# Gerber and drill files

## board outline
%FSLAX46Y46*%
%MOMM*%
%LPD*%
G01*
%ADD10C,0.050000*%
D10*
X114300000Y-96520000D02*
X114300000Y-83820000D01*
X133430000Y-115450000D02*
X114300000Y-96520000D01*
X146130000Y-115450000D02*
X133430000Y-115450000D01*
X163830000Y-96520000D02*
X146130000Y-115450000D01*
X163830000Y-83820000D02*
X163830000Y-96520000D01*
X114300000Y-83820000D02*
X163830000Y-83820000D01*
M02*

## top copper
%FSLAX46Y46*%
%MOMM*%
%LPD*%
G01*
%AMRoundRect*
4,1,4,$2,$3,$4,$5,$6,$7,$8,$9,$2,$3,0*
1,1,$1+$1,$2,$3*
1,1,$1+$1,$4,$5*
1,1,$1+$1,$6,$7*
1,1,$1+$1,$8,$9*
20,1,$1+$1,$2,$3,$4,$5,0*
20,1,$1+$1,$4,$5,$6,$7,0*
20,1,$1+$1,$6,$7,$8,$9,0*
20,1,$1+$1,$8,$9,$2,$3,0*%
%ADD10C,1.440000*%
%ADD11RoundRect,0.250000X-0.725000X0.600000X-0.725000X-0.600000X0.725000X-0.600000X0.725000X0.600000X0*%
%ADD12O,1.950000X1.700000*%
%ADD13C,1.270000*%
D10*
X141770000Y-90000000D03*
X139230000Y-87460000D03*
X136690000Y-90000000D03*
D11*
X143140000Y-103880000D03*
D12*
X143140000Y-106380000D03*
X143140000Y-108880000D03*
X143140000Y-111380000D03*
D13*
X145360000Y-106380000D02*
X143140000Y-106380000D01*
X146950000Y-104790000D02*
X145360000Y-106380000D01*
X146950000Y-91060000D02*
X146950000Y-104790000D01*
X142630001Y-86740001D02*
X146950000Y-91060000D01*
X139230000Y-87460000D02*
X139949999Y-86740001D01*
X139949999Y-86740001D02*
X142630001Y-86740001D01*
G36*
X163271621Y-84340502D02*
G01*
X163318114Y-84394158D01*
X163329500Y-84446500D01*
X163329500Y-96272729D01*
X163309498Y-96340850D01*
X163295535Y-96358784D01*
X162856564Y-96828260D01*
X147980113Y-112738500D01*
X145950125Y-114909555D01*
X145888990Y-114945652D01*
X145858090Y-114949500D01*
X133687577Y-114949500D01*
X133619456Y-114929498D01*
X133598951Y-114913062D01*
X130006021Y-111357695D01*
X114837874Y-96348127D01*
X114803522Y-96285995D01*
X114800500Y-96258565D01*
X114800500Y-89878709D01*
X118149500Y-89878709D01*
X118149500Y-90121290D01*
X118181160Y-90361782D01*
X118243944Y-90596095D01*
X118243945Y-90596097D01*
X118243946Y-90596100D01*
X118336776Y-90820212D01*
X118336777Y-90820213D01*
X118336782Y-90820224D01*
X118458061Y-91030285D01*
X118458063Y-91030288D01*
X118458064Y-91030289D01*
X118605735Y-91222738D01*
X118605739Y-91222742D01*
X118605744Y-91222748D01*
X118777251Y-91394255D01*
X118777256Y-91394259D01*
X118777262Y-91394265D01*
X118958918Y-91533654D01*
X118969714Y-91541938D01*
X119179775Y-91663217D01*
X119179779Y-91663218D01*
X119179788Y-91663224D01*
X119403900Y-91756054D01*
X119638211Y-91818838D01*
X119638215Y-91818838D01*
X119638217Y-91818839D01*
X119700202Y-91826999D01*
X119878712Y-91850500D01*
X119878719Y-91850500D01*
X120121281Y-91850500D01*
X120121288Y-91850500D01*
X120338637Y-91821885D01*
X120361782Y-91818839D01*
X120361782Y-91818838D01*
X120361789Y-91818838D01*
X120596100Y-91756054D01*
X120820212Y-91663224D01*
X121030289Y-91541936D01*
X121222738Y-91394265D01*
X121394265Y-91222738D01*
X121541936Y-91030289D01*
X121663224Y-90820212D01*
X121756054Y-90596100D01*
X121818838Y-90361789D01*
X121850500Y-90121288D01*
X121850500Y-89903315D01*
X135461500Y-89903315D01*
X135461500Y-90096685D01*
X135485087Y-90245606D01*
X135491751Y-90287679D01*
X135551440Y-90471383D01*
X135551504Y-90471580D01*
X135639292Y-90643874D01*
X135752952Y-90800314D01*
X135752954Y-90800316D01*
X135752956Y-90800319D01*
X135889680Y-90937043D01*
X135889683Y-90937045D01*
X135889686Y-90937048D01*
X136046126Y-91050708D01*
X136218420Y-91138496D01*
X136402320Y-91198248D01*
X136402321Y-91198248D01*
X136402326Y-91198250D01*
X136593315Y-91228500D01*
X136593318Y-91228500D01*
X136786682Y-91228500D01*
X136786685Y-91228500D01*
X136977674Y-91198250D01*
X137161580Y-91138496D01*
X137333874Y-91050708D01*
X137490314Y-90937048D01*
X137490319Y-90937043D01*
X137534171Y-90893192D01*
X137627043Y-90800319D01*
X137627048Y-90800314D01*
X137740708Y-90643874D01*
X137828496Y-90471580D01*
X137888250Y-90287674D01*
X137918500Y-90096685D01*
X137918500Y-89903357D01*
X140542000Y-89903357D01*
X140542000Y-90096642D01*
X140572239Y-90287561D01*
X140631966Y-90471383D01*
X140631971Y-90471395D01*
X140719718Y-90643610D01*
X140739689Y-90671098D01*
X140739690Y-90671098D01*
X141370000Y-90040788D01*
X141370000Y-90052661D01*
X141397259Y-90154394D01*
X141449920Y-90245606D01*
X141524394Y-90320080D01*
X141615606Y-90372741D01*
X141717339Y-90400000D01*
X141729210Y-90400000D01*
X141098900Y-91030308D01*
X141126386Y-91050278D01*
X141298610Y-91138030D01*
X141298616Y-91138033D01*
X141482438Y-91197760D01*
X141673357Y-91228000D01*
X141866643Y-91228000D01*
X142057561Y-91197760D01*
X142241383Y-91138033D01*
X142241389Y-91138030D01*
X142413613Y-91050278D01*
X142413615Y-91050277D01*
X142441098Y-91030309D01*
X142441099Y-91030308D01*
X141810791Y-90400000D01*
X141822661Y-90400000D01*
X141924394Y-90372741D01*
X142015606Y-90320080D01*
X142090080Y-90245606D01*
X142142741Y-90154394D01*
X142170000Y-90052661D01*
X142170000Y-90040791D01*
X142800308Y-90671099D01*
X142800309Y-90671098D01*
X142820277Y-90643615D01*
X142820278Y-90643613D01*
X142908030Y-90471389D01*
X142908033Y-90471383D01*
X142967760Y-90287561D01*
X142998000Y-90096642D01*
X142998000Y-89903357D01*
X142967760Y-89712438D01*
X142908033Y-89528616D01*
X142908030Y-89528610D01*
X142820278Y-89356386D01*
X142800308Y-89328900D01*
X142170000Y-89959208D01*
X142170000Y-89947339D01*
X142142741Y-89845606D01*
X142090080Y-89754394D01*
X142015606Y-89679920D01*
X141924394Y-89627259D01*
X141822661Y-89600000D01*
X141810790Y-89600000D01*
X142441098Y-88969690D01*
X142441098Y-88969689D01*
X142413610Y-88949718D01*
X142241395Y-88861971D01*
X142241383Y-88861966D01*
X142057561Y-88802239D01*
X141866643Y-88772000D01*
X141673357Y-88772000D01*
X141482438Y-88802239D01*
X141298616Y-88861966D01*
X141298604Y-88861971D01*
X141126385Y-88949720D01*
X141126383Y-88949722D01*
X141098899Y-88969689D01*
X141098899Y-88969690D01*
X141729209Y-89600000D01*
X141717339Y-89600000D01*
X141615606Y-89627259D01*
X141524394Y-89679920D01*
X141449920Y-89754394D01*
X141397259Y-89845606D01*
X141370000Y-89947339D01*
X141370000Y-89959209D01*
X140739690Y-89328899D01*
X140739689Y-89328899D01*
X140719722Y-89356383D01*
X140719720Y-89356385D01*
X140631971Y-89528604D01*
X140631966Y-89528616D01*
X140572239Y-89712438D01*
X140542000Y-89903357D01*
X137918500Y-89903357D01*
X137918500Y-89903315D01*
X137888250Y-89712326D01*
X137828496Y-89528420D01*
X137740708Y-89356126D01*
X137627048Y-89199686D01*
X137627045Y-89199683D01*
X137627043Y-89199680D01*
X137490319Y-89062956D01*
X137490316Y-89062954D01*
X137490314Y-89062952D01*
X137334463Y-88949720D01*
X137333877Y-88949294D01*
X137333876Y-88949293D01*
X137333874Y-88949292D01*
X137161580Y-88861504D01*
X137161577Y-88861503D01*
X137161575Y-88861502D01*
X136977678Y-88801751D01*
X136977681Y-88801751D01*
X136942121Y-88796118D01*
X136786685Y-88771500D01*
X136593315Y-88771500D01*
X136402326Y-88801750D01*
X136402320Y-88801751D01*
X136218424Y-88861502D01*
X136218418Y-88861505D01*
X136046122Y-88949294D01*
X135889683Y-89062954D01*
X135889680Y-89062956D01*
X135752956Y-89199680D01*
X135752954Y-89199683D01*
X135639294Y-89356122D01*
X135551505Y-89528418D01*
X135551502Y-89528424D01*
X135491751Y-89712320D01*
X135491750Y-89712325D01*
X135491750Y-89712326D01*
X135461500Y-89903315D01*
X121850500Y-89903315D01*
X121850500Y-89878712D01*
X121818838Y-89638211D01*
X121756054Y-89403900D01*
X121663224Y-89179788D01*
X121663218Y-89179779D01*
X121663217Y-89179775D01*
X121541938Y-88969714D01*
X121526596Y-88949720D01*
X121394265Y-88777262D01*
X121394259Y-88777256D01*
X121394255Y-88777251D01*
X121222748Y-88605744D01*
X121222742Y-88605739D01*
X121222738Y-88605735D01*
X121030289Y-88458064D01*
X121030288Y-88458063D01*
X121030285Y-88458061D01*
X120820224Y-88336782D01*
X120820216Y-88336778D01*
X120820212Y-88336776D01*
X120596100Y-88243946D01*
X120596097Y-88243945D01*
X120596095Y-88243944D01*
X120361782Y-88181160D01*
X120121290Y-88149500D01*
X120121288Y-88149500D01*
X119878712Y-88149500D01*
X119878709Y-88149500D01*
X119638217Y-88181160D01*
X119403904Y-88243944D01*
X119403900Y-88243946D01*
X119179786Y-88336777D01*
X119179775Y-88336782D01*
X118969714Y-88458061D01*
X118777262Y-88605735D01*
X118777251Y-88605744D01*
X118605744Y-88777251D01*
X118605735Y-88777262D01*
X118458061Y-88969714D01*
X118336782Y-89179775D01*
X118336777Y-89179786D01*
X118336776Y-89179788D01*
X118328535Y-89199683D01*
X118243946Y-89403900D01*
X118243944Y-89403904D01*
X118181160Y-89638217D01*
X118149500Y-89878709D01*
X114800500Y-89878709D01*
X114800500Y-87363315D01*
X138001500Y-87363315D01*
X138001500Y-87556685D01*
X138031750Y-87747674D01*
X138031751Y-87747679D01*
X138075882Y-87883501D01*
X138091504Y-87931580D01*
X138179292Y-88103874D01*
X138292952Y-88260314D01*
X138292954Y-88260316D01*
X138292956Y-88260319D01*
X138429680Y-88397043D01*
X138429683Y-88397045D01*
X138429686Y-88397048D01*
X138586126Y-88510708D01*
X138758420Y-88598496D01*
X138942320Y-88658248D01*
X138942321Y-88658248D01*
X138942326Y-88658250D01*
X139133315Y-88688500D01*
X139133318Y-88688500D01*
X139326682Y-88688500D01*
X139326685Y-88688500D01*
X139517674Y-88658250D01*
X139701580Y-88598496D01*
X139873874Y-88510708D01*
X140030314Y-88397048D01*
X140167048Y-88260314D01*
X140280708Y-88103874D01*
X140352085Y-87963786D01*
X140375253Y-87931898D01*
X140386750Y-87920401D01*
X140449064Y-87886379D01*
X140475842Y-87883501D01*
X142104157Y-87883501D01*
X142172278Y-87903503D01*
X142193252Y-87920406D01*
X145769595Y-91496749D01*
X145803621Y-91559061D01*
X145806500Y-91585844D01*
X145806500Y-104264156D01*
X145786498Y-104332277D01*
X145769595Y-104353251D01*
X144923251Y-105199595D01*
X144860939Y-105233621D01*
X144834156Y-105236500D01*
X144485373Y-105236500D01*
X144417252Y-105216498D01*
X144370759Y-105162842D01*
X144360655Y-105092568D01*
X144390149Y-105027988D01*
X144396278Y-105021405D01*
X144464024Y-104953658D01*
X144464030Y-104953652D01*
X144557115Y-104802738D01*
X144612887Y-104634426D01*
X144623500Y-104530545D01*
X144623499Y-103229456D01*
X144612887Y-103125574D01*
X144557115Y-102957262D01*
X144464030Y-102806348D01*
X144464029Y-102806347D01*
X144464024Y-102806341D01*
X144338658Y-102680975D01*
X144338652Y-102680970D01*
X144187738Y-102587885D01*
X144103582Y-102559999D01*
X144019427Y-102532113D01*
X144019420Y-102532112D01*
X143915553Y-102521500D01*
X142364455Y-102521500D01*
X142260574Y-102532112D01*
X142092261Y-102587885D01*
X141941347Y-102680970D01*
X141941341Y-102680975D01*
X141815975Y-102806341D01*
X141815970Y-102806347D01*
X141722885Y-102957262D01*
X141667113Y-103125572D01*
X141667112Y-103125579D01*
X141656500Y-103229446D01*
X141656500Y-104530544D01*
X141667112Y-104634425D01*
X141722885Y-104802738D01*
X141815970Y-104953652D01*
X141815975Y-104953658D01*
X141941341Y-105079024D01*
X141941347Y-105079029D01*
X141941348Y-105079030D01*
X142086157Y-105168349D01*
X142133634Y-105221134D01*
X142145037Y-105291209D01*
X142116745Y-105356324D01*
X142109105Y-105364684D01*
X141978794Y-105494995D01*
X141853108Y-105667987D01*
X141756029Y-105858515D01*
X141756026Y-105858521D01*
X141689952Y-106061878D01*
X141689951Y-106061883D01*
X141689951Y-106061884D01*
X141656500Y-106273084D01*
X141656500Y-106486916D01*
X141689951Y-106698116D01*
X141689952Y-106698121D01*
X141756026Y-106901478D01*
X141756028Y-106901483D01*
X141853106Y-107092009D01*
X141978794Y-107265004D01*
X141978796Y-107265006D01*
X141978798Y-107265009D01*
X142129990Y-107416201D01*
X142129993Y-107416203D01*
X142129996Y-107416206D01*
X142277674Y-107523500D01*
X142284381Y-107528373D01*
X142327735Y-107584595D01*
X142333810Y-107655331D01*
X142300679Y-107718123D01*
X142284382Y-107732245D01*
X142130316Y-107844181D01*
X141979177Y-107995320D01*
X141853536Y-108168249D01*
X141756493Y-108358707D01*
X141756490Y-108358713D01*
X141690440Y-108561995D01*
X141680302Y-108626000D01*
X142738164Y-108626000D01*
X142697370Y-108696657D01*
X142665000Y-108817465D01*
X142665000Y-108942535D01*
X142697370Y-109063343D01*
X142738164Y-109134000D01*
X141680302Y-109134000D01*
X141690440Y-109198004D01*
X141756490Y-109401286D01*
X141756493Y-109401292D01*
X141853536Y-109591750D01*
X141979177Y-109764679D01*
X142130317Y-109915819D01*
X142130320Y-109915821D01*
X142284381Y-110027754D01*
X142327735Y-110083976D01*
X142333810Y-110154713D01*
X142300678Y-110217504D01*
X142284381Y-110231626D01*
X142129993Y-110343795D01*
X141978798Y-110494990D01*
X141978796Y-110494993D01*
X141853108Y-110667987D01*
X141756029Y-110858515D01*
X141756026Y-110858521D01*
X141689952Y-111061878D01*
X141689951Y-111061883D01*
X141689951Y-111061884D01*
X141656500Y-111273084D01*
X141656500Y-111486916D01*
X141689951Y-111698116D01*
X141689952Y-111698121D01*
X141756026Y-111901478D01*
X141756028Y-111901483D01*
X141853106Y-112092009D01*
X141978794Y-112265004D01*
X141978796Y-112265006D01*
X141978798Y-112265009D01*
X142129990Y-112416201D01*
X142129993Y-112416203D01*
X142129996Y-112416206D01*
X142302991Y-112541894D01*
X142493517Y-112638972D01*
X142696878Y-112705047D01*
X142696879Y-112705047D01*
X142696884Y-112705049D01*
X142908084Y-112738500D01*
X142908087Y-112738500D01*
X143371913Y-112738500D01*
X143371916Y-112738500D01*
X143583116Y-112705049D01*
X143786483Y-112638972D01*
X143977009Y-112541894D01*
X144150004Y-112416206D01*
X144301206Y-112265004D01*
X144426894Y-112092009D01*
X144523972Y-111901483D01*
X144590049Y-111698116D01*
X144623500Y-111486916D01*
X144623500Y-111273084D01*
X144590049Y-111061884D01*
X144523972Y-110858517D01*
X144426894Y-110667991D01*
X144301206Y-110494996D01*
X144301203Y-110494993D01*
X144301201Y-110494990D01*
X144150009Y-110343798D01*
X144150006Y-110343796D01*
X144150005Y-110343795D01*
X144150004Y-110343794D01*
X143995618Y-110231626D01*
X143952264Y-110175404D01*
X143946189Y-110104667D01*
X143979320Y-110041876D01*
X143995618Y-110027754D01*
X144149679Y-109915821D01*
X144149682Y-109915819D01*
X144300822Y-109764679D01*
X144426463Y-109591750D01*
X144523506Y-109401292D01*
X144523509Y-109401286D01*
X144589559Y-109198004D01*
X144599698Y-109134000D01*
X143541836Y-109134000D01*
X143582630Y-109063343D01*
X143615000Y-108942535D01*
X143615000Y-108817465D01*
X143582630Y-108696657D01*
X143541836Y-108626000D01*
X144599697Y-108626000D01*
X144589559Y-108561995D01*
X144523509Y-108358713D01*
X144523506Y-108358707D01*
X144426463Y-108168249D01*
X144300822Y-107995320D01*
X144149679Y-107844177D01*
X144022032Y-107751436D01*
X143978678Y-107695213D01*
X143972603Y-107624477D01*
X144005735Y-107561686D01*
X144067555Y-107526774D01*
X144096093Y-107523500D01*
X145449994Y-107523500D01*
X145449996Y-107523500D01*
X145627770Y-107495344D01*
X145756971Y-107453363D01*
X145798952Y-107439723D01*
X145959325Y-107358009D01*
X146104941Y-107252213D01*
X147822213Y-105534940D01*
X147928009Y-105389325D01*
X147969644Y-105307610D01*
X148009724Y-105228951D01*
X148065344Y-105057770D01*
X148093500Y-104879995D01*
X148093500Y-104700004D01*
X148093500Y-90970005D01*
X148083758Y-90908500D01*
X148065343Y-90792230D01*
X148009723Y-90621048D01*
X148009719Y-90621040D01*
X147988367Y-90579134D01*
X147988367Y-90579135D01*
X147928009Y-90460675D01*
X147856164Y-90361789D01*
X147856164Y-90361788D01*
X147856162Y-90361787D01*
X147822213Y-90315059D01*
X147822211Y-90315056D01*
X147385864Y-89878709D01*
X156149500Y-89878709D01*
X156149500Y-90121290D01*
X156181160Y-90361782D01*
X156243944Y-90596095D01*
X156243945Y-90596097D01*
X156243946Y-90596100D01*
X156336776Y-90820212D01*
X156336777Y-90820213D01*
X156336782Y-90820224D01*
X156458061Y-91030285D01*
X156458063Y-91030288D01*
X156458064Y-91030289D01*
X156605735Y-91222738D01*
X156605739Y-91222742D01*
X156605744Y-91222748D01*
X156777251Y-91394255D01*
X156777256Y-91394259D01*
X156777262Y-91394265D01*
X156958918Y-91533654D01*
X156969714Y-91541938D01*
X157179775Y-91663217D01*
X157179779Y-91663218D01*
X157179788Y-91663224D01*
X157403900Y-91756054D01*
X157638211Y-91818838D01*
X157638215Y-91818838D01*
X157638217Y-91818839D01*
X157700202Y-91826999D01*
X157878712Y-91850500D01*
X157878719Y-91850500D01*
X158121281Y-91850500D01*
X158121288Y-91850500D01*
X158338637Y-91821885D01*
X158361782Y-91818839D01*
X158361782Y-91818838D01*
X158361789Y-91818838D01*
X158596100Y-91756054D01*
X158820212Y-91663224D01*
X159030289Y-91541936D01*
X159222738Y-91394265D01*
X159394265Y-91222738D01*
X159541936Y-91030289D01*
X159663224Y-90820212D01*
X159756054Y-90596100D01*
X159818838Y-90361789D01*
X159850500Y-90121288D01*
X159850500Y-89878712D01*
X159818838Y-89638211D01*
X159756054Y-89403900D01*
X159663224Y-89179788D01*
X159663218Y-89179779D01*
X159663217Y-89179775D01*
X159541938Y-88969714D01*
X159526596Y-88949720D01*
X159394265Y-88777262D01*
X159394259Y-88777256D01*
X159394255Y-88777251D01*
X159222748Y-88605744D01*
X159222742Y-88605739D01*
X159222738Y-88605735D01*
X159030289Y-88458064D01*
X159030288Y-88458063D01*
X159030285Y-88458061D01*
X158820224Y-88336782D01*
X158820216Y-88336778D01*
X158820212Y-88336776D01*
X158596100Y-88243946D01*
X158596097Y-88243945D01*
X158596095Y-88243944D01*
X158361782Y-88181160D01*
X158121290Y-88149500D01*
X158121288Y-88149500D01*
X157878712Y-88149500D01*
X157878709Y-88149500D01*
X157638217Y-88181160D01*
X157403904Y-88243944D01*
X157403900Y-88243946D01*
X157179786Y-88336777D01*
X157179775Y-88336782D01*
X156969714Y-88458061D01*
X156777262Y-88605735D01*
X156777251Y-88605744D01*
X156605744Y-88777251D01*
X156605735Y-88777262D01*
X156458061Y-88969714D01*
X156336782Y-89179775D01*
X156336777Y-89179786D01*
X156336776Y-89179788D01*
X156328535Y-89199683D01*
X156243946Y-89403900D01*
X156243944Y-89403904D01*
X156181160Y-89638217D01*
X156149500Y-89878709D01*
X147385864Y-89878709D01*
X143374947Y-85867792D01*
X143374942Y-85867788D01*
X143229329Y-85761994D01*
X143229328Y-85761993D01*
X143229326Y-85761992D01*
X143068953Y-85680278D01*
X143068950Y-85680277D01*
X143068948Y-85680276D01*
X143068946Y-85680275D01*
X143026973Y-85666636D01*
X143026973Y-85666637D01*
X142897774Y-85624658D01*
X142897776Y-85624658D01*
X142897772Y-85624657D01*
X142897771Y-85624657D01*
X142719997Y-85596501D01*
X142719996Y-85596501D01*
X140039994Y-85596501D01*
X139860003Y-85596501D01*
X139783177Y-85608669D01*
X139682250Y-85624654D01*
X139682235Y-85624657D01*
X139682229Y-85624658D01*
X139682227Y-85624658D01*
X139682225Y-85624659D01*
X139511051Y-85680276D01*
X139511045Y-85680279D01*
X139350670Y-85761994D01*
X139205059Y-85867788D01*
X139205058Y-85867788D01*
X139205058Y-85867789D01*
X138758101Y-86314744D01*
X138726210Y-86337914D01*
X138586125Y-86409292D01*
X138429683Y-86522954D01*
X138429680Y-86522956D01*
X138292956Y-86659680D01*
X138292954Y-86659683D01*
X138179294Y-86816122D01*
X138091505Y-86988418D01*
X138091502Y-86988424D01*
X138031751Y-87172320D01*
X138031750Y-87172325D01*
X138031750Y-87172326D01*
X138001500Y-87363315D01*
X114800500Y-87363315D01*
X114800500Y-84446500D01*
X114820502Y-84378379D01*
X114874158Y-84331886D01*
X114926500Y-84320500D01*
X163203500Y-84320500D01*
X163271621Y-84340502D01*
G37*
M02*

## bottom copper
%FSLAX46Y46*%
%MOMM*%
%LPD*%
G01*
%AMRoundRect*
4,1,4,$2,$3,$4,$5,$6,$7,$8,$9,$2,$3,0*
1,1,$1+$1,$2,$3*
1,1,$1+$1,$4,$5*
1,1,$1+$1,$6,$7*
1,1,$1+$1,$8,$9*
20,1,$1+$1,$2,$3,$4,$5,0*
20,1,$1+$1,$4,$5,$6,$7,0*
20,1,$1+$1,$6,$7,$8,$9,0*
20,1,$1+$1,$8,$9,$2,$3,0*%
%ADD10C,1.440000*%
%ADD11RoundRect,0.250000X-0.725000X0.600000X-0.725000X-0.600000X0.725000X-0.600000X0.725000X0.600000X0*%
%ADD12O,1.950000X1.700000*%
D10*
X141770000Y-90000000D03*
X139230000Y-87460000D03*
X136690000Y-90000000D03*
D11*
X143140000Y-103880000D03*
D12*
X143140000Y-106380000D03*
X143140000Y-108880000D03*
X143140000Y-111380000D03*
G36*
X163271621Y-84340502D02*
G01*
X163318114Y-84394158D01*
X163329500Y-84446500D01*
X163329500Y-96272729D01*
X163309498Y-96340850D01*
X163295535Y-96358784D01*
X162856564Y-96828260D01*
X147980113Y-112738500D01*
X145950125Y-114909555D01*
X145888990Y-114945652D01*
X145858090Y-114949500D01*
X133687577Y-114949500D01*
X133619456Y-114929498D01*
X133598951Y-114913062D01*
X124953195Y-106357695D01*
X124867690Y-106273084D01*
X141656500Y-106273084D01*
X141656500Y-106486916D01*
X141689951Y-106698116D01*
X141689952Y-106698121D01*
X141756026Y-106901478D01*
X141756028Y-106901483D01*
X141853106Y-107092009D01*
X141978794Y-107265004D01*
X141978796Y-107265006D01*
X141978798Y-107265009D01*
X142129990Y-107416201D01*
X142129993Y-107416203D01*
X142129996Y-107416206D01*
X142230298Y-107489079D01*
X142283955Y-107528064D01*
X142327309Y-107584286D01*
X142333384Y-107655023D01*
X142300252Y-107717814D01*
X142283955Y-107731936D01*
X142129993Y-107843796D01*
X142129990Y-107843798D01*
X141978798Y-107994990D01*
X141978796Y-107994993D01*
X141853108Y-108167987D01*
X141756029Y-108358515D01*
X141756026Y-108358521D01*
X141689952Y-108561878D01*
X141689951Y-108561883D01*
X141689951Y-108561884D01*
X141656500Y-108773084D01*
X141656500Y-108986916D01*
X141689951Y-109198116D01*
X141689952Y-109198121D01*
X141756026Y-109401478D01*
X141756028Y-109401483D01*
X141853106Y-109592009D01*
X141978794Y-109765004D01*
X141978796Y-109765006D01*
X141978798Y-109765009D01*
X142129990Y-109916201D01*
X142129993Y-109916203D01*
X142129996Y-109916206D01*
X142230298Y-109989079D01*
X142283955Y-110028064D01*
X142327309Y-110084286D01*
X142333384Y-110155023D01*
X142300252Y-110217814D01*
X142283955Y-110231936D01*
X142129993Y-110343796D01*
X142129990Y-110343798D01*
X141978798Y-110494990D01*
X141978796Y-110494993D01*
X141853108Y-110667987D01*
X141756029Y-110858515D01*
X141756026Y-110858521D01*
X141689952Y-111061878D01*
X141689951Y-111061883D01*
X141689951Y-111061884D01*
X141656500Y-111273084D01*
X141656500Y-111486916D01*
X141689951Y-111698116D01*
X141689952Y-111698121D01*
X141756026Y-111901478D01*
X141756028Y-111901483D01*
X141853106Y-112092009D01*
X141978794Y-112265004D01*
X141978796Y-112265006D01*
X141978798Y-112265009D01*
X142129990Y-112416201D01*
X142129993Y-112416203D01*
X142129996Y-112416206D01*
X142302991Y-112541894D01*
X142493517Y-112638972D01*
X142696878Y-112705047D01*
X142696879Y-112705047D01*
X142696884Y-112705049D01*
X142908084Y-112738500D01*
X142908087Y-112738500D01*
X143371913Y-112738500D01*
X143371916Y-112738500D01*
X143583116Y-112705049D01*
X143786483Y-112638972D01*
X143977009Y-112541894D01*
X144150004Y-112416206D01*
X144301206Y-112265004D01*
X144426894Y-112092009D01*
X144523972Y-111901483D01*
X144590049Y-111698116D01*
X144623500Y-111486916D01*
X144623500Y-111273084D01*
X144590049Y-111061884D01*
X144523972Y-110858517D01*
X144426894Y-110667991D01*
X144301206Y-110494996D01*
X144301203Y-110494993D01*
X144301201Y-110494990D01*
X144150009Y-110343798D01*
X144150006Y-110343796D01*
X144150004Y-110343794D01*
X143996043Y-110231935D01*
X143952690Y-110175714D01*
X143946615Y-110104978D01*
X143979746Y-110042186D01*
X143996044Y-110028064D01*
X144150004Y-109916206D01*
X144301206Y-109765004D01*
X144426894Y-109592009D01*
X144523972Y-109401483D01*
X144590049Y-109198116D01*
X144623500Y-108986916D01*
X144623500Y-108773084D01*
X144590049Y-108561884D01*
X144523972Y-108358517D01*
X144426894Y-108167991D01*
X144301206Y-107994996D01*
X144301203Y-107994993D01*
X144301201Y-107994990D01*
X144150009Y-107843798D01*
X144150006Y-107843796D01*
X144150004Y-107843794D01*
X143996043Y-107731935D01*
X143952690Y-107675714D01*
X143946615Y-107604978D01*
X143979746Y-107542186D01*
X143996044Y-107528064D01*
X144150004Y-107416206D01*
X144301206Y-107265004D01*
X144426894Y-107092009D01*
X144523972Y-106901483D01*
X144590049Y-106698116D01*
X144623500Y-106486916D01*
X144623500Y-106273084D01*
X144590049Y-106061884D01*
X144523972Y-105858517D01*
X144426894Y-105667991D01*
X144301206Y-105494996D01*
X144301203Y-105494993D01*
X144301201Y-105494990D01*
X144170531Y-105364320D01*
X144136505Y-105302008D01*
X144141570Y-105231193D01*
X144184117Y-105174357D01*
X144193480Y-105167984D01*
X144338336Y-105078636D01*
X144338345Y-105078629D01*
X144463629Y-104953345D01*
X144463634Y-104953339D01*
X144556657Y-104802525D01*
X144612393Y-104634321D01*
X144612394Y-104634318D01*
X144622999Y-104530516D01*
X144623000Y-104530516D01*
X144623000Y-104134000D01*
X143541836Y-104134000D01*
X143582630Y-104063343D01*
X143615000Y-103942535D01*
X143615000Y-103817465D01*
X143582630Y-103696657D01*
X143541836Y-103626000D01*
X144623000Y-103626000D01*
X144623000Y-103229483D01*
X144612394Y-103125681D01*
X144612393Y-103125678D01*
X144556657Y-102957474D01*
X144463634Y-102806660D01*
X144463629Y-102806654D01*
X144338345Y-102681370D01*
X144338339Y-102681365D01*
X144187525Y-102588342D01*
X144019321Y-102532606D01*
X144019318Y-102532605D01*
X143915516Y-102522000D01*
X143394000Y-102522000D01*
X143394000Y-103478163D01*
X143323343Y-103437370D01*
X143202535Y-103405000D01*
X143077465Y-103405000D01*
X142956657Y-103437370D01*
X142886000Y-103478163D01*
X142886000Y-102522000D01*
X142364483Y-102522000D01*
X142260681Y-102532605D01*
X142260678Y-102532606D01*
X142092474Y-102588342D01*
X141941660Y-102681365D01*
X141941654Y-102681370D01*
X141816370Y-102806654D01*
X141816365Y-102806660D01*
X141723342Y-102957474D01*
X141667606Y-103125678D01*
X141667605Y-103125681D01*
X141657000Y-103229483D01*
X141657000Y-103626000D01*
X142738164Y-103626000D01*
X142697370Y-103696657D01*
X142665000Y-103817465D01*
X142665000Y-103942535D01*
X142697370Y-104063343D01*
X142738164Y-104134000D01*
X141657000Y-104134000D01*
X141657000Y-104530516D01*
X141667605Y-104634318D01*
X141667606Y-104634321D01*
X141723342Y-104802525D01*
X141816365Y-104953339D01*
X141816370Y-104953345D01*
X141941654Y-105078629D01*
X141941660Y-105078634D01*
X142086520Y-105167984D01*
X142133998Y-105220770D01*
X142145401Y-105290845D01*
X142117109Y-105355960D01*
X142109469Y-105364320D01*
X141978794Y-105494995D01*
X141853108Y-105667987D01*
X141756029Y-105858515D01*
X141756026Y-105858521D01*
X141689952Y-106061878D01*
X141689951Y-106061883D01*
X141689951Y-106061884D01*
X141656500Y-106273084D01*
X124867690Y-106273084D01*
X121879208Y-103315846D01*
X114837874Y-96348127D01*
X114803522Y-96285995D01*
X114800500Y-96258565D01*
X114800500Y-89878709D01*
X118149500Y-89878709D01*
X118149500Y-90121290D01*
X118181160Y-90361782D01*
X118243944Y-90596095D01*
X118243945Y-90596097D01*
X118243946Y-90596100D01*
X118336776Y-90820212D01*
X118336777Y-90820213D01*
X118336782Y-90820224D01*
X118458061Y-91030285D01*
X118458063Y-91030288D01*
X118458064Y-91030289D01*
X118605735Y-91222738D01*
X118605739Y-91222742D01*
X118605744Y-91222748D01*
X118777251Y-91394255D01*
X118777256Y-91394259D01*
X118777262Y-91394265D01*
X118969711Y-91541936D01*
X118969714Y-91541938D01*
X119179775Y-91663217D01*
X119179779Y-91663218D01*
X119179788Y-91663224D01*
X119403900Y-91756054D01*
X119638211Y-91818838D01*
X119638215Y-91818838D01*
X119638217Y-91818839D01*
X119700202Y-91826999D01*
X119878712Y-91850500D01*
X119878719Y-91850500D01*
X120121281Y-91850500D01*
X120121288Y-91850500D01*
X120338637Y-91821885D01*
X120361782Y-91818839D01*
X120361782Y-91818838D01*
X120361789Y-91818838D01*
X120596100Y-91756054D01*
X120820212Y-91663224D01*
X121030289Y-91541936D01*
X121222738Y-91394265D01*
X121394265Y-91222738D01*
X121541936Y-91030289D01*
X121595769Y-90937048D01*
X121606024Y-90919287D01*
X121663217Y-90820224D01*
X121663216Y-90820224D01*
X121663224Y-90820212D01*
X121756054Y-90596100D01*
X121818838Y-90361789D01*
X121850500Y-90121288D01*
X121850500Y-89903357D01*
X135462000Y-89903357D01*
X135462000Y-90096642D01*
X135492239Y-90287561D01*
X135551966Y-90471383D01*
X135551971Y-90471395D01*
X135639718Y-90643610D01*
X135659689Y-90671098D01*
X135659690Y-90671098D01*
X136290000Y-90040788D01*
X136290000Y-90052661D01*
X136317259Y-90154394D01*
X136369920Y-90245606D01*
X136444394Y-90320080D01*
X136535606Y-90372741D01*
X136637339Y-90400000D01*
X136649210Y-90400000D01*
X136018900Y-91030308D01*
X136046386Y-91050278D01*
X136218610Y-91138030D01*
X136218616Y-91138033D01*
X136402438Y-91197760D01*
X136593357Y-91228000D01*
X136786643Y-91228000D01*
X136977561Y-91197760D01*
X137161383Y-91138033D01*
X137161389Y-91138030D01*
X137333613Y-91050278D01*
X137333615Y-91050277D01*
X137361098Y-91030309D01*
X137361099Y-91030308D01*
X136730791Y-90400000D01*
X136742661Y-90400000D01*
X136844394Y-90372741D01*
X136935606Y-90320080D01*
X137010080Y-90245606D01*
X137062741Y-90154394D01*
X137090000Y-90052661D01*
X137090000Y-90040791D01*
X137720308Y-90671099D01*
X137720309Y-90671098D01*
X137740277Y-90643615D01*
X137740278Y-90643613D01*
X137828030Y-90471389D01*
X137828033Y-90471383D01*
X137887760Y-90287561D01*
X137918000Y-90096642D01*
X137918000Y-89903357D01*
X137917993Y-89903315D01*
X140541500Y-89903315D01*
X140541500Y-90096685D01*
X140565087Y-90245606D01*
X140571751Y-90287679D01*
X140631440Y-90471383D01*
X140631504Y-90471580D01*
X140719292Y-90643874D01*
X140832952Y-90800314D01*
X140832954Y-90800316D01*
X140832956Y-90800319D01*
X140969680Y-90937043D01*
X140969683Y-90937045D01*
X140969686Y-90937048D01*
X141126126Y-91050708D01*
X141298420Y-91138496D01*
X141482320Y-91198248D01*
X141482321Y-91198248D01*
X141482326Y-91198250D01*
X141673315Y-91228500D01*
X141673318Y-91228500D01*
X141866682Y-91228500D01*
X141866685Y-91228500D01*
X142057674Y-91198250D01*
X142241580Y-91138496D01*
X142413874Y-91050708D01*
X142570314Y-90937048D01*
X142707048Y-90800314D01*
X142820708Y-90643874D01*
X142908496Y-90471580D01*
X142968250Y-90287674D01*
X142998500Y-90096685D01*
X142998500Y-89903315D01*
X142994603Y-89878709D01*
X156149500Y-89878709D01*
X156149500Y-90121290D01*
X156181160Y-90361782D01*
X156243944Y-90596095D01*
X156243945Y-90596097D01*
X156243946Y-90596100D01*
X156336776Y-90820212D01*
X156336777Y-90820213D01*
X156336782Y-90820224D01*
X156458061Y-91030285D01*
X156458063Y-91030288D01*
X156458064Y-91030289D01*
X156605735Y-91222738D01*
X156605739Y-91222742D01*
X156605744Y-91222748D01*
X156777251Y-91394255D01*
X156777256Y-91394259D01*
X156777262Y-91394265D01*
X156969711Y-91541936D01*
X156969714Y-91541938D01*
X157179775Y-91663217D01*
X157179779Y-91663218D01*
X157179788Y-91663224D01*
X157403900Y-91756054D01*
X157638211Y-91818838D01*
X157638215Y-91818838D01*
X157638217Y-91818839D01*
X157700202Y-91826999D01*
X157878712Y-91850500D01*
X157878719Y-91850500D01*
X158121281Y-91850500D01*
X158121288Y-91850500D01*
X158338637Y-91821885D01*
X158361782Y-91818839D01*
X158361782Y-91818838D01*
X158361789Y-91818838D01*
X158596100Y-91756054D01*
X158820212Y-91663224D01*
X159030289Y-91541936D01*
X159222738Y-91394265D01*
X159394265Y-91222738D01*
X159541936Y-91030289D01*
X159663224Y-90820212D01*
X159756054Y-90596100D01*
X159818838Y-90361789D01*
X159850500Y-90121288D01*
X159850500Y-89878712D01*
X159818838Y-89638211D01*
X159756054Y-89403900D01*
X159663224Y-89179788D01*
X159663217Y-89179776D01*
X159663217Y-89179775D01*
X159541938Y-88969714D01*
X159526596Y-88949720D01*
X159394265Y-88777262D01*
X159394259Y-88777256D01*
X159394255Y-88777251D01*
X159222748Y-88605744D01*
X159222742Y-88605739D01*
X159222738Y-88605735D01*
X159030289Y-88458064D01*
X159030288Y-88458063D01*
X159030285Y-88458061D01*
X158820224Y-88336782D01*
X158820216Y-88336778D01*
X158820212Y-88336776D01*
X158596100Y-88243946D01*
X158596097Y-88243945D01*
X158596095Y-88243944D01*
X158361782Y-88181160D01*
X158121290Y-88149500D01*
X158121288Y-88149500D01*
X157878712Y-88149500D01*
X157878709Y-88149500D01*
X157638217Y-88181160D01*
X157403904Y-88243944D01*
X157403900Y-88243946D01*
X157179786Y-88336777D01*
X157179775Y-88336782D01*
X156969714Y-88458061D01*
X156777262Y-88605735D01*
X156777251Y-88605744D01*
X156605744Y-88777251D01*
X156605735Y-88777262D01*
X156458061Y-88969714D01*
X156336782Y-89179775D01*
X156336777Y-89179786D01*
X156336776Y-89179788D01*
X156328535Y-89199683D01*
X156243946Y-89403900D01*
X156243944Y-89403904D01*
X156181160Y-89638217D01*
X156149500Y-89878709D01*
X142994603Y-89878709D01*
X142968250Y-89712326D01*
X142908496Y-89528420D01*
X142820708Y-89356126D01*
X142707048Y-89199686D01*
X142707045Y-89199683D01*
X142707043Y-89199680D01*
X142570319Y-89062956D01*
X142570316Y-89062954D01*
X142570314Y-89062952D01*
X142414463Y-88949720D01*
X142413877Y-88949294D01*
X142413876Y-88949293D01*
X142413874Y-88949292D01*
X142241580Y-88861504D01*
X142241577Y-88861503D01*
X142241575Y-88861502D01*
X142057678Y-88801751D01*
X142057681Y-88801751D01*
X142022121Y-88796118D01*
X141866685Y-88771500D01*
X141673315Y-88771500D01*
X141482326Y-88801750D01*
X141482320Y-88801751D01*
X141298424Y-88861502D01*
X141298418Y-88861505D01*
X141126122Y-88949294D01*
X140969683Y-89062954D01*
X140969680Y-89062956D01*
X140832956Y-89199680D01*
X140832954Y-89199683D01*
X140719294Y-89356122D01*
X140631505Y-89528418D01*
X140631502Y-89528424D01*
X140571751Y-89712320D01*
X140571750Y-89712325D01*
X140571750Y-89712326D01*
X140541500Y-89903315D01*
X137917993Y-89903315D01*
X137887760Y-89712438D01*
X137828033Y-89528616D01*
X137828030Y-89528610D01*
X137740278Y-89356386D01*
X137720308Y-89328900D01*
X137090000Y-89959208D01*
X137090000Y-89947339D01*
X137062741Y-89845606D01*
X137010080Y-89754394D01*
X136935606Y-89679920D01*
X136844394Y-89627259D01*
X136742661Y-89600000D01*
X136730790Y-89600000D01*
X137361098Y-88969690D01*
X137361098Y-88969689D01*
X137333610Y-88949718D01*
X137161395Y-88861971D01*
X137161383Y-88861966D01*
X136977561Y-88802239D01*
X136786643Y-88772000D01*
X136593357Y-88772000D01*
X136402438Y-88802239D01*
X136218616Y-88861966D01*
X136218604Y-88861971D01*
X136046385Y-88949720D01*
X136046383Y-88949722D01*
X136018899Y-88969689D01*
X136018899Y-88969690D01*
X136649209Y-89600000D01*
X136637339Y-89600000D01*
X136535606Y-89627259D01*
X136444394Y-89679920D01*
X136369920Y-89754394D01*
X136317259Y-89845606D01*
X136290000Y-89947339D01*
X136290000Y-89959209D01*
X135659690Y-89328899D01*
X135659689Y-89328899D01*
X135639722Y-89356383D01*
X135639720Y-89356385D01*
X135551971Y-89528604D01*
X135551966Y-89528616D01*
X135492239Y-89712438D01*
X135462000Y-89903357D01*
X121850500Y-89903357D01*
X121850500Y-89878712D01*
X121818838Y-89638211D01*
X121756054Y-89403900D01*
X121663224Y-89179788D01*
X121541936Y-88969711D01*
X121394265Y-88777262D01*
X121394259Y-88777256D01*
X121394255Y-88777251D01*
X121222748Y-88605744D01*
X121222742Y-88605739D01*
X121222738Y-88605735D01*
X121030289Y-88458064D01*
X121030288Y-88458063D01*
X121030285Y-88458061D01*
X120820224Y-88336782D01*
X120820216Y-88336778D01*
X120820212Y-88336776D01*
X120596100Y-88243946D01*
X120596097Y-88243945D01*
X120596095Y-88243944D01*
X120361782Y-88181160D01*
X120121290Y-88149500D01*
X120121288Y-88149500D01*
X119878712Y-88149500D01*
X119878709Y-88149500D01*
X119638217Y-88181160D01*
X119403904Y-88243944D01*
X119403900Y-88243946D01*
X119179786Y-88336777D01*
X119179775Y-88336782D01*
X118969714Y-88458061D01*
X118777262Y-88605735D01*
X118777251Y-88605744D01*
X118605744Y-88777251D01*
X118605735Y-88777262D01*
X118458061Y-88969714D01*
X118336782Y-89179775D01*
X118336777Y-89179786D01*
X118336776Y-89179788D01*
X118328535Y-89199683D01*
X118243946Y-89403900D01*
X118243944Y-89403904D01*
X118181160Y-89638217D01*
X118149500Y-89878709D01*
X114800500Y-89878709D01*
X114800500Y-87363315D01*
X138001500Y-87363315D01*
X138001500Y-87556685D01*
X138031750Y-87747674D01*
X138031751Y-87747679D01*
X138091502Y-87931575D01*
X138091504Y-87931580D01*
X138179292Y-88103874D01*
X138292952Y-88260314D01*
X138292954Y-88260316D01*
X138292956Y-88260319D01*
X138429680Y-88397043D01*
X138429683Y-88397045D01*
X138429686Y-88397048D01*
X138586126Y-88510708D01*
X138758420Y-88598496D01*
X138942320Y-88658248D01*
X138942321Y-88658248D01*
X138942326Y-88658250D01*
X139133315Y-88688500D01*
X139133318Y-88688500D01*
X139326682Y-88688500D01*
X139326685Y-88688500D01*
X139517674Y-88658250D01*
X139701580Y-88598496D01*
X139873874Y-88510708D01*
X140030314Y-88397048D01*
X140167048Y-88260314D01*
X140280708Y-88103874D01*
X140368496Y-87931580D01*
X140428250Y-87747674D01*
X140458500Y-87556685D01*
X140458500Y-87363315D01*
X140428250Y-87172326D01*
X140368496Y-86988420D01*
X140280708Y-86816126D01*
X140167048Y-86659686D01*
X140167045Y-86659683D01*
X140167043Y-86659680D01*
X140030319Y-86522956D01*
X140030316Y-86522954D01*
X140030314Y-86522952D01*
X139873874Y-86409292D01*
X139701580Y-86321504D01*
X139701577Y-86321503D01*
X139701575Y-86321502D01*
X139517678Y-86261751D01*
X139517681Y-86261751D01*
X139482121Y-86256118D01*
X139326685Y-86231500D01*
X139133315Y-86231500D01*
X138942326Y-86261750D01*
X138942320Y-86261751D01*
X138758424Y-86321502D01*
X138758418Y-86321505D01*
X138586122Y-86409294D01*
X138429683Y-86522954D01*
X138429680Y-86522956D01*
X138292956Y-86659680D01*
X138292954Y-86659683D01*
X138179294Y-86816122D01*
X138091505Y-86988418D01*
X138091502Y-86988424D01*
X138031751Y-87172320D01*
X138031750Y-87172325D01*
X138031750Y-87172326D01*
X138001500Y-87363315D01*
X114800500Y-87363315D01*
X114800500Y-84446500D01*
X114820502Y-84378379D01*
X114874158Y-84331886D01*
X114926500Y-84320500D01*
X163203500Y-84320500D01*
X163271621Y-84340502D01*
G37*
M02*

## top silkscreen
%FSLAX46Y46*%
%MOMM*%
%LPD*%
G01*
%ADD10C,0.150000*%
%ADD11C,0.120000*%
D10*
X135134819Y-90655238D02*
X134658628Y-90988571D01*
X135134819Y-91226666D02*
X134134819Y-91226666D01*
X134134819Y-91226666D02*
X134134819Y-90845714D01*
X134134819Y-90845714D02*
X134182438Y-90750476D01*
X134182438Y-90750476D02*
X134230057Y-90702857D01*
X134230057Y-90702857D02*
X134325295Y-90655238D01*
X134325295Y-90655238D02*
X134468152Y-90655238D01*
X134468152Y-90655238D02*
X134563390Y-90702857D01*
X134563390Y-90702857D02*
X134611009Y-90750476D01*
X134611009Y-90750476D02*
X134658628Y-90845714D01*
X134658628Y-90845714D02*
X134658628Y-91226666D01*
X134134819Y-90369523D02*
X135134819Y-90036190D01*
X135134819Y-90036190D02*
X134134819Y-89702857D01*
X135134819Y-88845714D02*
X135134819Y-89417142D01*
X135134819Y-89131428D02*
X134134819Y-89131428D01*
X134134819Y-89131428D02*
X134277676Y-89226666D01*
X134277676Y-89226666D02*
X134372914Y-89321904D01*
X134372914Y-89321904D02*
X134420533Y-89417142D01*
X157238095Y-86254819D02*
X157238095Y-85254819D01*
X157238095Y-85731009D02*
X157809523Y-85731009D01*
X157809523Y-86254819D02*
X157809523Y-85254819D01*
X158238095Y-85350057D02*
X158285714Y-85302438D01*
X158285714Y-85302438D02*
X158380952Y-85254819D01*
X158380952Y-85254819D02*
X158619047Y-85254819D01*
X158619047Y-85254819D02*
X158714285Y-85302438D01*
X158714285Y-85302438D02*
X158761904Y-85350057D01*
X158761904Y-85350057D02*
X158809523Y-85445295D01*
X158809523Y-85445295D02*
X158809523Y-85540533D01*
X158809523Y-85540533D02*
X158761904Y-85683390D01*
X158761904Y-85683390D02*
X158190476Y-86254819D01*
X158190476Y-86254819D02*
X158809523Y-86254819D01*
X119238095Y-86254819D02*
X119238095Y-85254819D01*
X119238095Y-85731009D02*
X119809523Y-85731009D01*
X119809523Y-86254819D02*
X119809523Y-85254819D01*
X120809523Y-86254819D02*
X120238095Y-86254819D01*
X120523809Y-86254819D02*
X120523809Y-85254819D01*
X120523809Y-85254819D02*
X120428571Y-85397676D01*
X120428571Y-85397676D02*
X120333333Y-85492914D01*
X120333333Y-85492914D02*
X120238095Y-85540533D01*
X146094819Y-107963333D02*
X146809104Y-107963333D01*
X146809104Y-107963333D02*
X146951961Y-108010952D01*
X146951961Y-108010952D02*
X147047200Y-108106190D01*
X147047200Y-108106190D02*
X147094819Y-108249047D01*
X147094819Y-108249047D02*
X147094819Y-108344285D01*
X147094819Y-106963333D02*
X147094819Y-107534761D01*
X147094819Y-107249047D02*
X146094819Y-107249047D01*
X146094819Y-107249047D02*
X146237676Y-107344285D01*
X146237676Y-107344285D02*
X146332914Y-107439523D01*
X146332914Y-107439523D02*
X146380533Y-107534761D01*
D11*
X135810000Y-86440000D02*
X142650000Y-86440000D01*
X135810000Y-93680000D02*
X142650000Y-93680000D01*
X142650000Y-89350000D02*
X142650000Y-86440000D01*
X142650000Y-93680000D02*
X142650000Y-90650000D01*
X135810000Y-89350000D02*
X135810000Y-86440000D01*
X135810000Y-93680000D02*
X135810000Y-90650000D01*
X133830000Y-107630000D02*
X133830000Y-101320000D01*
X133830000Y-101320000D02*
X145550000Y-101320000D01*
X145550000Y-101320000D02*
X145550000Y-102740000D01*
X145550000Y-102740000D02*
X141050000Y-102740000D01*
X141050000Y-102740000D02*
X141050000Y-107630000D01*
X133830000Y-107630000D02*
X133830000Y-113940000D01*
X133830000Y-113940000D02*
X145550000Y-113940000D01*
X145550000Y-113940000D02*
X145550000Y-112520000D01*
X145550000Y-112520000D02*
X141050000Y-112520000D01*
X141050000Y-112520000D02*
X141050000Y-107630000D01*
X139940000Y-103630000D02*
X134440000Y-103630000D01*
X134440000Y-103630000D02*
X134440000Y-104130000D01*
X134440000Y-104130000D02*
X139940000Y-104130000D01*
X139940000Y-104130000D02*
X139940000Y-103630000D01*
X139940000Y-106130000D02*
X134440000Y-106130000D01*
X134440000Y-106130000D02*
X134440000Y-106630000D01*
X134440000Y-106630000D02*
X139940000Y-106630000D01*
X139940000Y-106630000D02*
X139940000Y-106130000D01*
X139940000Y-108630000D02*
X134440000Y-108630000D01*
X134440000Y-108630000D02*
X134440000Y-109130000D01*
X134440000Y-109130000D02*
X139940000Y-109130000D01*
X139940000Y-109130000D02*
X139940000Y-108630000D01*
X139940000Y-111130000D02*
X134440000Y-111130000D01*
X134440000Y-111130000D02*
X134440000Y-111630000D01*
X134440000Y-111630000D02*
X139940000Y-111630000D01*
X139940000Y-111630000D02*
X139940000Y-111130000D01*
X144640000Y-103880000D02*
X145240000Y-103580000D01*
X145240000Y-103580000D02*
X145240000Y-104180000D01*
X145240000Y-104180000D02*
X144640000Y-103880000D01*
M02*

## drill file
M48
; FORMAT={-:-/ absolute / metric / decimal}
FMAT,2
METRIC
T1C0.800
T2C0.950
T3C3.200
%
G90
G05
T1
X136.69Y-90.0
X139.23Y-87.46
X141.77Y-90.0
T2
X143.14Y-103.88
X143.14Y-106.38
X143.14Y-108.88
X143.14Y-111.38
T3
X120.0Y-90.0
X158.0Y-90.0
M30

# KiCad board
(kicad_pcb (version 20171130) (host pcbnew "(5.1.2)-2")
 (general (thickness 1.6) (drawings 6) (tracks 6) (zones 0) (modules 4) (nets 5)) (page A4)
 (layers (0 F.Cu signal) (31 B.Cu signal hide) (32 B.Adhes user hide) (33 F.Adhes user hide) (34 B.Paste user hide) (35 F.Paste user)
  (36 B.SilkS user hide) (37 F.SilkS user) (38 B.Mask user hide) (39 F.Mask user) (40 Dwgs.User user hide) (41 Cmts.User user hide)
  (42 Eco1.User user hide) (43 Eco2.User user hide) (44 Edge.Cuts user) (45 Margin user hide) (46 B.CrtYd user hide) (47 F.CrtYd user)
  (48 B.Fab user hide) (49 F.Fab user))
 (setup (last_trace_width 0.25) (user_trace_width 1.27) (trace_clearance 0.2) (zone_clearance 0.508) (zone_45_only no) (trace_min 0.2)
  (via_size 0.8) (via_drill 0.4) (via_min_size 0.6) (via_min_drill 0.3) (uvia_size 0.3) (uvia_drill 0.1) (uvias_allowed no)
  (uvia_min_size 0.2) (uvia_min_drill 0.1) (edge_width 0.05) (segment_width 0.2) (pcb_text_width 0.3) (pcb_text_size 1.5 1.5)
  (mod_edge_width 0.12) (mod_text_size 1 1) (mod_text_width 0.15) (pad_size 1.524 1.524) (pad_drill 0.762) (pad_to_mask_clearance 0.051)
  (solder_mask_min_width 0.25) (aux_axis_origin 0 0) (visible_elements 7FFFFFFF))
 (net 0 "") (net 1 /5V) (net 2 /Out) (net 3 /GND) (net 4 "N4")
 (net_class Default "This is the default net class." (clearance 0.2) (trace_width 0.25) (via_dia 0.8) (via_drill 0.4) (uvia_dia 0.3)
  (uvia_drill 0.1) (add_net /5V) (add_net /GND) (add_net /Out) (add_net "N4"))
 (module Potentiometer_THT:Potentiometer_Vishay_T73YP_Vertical (layer F.Cu) (at 141.77 90 90)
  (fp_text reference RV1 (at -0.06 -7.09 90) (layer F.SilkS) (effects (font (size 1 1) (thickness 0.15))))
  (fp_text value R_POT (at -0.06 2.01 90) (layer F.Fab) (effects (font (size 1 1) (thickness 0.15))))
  (fp_line (start 3.56 -5.96) (end 3.56 0.88) (layer F.SilkS) (width 0.12))
  (fp_line (start -3.68 -5.96) (end -3.68 0.88) (layer F.SilkS) (width 0.12))
  (fp_line (start 0.65 0.88) (end 3.56 0.88) (layer F.SilkS) (width 0.12))
  (fp_line (start -3.68 0.88) (end -0.65 0.88) (layer F.SilkS) (width 0.12))
  (fp_line (start 0.65 -5.96) (end 3.56 -5.96) (layer F.SilkS) (width 0.12))
  (fp_line (start -3.68 -5.96) (end -0.65 -5.96) (layer F.SilkS) (width 0.12))
  (pad 1 thru_hole circle (at 0 0 90) (size 1.44 1.44) (drill 0.8) (layers *.Cu *.Mask) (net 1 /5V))
  (pad 2 thru_hole circle (at 2.54 -2.54 90) (size 1.44 1.44) (drill 0.8) (layers *.Cu *.Mask) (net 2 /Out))
  (pad 3 thru_hole circle (at 0 -5.08 90) (size 1.44 1.44) (drill 0.8) (layers *.Cu *.Mask) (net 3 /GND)))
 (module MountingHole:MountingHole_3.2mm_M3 (layer F.Cu) (at 158 90)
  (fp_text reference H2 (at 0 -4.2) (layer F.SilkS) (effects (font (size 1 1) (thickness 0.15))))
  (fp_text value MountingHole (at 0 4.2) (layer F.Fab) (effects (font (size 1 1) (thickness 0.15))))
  (pad 1 np_thru_hole circle (at 0 0) (size 3.2 3.2) (drill 3.2) (layers *.Cu *.Mask)))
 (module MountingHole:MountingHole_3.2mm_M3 (layer F.Cu) (at 120 90)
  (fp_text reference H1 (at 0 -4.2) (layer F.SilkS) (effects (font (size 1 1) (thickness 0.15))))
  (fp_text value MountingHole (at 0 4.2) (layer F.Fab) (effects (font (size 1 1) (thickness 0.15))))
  (pad 1 np_thru_hole circle (at 0 0) (size 3.2 3.2) (drill 3.2) (layers *.Cu *.Mask)))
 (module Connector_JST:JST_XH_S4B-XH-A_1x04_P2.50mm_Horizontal (layer F.Cu) (at 143.14 103.88 270)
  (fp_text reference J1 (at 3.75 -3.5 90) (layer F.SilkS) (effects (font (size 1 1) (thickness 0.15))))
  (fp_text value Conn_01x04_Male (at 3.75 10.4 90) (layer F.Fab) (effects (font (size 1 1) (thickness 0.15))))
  (fp_line (start 3.75 9.31) (end -2.56 9.31) (layer F.SilkS) (width 0.12))
  (fp_line (start -2.56 9.31) (end -2.56 -2.41) (layer F.SilkS) (width 0.12))
  (fp_line (start -2.56 -2.41) (end -1.14 -2.41) (layer F.SilkS) (width 0.12))
  (fp_line (start -1.14 -2.41) (end -1.14 2.09) (layer F.SilkS) (width 0.12))
  (fp_line (start -1.14 2.09) (end 3.75 2.09) (layer F.SilkS) (width 0.12))
  (fp_line (start 3.75 9.31) (end 10.06 9.31) (layer F.SilkS) (width 0.12))
  (fp_line (start 10.06 9.31) (end 10.06 -2.41) (layer F.SilkS) (width 0.12))
  (fp_line (start 10.06 -2.41) (end 8.64 -2.41) (layer F.SilkS) (width 0.12))
  (fp_line (start 8.64 -2.41) (end 8.64 2.09) (layer F.SilkS) (width 0.12))
  (fp_line (start 8.64 2.09) (end 3.75 2.09) (layer F.SilkS) (width 0.12))
  (fp_line (start -0.25 3.2) (end -0.25 8.7) (layer F.SilkS) (width 0.12))
  (fp_line (start -0.25 8.7) (end 0.25 8.7) (layer F.SilkS) (width 0.12))
  (fp_line (start 0.25 8.7) (end 0.25 3.2) (layer F.SilkS) (width 0.12))
  (fp_line (start 0.25 3.2) (end -0.25 3.2) (layer F.SilkS) (width 0.12))
  (fp_line (start 2.25 3.2) (end 2.25 8.7) (layer F.SilkS) (width 0.12))
  (fp_line (start 2.25 8.7) (end 2.75 8.7) (layer F.SilkS) (width 0.12))
  (fp_line (start 2.75 8.7) (end 2.75 3.2) (layer F.SilkS) (width 0.12))
  (fp_line (start 2.75 3.2) (end 2.25 3.2) (layer F.SilkS) (width 0.12))
  (fp_line (start 4.75 3.2) (end 4.75 8.7) (layer F.SilkS) (width 0.12))
  (fp_line (start 4.75 8.7) (end 5.25 8.7) (layer F.SilkS) (width 0.12))
  (fp_line (start 5.25 8.7) (end 5.25 3.2) (layer F.SilkS) (width 0.12))
  (fp_line (start 5.25 3.2) (end 4.75 3.2) (layer F.SilkS) (width 0.12))
  (fp_line (start 7.25 3.2) (end 7.25 8.7) (layer F.SilkS) (width 0.12))
  (fp_line (start 7.25 8.7) (end 7.75 8.7) (layer F.SilkS) (width 0.12))
  (fp_line (start 7.75 8.7) (end 7.75 3.2) (layer F.SilkS) (width 0.12))
  (fp_line (start 7.75 3.2) (end 7.25 3.2) (layer F.SilkS) (width 0.12))
  (fp_line (start 0 -1.5) (end -0.3 -2.1) (layer F.SilkS) (width 0.12))
  (fp_line (start -0.3 -2.1) (end 0.3 -2.1) (layer F.SilkS) (width 0.12))
  (fp_line (start 0.3 -2.1) (end 0 -1.5) (layer F.SilkS) (width 0.12))
  (pad 1 thru_hole roundrect (at 0 0 270) (size 1.7 1.95) (drill 0.95) (layers *.Cu *.Mask) (roundrect_rratio 0.147059) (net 3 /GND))
  (pad 2 thru_hole oval (at 2.5 0 270) (size 1.7 1.95) (drill 0.95) (layers *.Cu *.Mask) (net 2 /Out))
  (pad 3 thru_hole oval (at 5 0 270) (size 1.7 1.95) (drill 0.95) (layers *.Cu *.Mask) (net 1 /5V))
  (pad 4 thru_hole oval (at 7.5 0 270) (size 1.7 1.95) (drill 0.95) (layers *.Cu *.Mask) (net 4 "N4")))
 (gr_line (start 114.3 96.52) (end 114.3 83.82) (layer Edge.Cuts) (width 0.05))
 (gr_line (start 133.43 115.45) (end 114.3 96.52) (layer Edge.Cuts) (width 0.05))
 (gr_line (start 146.13 115.45) (end 133.43 115.45) (layer Edge.Cuts) (width 0.05))
 (gr_line (start 163.83 96.52) (end 146.13 115.45) (layer Edge.Cuts) (width 0.05))
 (gr_line (start 163.83 83.82) (end 163.83 96.52) (layer Edge.Cuts) (width 0.05))
 (gr_line (start 114.3 83.82) (end 163.83 83.82) (layer Edge.Cuts) (width 0.05))
 (segment (start 145.36 106.38) (end 143.14 106.38) (width 1.27) (layer F.Cu) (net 2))
 (segment (start 146.95 104.79) (end 145.36 106.38) (width 1.27) (layer F.Cu) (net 2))
 (segment (start 146.95 91.06) (end 146.95 104.79) (width 1.27) (layer F.Cu) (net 2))
 (segment (start 142.630001 86.740001) (end 146.95 91.06) (width 1.27) (layer F.Cu) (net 2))
 (segment (start 139.23 87.46) (end 139.949999 86.740001) (width 1.27) (layer F.Cu) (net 2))
 (segment (start 139.949999 86.740001) (end 142.630001 86.740001) (width 1.27) (layer F.Cu) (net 2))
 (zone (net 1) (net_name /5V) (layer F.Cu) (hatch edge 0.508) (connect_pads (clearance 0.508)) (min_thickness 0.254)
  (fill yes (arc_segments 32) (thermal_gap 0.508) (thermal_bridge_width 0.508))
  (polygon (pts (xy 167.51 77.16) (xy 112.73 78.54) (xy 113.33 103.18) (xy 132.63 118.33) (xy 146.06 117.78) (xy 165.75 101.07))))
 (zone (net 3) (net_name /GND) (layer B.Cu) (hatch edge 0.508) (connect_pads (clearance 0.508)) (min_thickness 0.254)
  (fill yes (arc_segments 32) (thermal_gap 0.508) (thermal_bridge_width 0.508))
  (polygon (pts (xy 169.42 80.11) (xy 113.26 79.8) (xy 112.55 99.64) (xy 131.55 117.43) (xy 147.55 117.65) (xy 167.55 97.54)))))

